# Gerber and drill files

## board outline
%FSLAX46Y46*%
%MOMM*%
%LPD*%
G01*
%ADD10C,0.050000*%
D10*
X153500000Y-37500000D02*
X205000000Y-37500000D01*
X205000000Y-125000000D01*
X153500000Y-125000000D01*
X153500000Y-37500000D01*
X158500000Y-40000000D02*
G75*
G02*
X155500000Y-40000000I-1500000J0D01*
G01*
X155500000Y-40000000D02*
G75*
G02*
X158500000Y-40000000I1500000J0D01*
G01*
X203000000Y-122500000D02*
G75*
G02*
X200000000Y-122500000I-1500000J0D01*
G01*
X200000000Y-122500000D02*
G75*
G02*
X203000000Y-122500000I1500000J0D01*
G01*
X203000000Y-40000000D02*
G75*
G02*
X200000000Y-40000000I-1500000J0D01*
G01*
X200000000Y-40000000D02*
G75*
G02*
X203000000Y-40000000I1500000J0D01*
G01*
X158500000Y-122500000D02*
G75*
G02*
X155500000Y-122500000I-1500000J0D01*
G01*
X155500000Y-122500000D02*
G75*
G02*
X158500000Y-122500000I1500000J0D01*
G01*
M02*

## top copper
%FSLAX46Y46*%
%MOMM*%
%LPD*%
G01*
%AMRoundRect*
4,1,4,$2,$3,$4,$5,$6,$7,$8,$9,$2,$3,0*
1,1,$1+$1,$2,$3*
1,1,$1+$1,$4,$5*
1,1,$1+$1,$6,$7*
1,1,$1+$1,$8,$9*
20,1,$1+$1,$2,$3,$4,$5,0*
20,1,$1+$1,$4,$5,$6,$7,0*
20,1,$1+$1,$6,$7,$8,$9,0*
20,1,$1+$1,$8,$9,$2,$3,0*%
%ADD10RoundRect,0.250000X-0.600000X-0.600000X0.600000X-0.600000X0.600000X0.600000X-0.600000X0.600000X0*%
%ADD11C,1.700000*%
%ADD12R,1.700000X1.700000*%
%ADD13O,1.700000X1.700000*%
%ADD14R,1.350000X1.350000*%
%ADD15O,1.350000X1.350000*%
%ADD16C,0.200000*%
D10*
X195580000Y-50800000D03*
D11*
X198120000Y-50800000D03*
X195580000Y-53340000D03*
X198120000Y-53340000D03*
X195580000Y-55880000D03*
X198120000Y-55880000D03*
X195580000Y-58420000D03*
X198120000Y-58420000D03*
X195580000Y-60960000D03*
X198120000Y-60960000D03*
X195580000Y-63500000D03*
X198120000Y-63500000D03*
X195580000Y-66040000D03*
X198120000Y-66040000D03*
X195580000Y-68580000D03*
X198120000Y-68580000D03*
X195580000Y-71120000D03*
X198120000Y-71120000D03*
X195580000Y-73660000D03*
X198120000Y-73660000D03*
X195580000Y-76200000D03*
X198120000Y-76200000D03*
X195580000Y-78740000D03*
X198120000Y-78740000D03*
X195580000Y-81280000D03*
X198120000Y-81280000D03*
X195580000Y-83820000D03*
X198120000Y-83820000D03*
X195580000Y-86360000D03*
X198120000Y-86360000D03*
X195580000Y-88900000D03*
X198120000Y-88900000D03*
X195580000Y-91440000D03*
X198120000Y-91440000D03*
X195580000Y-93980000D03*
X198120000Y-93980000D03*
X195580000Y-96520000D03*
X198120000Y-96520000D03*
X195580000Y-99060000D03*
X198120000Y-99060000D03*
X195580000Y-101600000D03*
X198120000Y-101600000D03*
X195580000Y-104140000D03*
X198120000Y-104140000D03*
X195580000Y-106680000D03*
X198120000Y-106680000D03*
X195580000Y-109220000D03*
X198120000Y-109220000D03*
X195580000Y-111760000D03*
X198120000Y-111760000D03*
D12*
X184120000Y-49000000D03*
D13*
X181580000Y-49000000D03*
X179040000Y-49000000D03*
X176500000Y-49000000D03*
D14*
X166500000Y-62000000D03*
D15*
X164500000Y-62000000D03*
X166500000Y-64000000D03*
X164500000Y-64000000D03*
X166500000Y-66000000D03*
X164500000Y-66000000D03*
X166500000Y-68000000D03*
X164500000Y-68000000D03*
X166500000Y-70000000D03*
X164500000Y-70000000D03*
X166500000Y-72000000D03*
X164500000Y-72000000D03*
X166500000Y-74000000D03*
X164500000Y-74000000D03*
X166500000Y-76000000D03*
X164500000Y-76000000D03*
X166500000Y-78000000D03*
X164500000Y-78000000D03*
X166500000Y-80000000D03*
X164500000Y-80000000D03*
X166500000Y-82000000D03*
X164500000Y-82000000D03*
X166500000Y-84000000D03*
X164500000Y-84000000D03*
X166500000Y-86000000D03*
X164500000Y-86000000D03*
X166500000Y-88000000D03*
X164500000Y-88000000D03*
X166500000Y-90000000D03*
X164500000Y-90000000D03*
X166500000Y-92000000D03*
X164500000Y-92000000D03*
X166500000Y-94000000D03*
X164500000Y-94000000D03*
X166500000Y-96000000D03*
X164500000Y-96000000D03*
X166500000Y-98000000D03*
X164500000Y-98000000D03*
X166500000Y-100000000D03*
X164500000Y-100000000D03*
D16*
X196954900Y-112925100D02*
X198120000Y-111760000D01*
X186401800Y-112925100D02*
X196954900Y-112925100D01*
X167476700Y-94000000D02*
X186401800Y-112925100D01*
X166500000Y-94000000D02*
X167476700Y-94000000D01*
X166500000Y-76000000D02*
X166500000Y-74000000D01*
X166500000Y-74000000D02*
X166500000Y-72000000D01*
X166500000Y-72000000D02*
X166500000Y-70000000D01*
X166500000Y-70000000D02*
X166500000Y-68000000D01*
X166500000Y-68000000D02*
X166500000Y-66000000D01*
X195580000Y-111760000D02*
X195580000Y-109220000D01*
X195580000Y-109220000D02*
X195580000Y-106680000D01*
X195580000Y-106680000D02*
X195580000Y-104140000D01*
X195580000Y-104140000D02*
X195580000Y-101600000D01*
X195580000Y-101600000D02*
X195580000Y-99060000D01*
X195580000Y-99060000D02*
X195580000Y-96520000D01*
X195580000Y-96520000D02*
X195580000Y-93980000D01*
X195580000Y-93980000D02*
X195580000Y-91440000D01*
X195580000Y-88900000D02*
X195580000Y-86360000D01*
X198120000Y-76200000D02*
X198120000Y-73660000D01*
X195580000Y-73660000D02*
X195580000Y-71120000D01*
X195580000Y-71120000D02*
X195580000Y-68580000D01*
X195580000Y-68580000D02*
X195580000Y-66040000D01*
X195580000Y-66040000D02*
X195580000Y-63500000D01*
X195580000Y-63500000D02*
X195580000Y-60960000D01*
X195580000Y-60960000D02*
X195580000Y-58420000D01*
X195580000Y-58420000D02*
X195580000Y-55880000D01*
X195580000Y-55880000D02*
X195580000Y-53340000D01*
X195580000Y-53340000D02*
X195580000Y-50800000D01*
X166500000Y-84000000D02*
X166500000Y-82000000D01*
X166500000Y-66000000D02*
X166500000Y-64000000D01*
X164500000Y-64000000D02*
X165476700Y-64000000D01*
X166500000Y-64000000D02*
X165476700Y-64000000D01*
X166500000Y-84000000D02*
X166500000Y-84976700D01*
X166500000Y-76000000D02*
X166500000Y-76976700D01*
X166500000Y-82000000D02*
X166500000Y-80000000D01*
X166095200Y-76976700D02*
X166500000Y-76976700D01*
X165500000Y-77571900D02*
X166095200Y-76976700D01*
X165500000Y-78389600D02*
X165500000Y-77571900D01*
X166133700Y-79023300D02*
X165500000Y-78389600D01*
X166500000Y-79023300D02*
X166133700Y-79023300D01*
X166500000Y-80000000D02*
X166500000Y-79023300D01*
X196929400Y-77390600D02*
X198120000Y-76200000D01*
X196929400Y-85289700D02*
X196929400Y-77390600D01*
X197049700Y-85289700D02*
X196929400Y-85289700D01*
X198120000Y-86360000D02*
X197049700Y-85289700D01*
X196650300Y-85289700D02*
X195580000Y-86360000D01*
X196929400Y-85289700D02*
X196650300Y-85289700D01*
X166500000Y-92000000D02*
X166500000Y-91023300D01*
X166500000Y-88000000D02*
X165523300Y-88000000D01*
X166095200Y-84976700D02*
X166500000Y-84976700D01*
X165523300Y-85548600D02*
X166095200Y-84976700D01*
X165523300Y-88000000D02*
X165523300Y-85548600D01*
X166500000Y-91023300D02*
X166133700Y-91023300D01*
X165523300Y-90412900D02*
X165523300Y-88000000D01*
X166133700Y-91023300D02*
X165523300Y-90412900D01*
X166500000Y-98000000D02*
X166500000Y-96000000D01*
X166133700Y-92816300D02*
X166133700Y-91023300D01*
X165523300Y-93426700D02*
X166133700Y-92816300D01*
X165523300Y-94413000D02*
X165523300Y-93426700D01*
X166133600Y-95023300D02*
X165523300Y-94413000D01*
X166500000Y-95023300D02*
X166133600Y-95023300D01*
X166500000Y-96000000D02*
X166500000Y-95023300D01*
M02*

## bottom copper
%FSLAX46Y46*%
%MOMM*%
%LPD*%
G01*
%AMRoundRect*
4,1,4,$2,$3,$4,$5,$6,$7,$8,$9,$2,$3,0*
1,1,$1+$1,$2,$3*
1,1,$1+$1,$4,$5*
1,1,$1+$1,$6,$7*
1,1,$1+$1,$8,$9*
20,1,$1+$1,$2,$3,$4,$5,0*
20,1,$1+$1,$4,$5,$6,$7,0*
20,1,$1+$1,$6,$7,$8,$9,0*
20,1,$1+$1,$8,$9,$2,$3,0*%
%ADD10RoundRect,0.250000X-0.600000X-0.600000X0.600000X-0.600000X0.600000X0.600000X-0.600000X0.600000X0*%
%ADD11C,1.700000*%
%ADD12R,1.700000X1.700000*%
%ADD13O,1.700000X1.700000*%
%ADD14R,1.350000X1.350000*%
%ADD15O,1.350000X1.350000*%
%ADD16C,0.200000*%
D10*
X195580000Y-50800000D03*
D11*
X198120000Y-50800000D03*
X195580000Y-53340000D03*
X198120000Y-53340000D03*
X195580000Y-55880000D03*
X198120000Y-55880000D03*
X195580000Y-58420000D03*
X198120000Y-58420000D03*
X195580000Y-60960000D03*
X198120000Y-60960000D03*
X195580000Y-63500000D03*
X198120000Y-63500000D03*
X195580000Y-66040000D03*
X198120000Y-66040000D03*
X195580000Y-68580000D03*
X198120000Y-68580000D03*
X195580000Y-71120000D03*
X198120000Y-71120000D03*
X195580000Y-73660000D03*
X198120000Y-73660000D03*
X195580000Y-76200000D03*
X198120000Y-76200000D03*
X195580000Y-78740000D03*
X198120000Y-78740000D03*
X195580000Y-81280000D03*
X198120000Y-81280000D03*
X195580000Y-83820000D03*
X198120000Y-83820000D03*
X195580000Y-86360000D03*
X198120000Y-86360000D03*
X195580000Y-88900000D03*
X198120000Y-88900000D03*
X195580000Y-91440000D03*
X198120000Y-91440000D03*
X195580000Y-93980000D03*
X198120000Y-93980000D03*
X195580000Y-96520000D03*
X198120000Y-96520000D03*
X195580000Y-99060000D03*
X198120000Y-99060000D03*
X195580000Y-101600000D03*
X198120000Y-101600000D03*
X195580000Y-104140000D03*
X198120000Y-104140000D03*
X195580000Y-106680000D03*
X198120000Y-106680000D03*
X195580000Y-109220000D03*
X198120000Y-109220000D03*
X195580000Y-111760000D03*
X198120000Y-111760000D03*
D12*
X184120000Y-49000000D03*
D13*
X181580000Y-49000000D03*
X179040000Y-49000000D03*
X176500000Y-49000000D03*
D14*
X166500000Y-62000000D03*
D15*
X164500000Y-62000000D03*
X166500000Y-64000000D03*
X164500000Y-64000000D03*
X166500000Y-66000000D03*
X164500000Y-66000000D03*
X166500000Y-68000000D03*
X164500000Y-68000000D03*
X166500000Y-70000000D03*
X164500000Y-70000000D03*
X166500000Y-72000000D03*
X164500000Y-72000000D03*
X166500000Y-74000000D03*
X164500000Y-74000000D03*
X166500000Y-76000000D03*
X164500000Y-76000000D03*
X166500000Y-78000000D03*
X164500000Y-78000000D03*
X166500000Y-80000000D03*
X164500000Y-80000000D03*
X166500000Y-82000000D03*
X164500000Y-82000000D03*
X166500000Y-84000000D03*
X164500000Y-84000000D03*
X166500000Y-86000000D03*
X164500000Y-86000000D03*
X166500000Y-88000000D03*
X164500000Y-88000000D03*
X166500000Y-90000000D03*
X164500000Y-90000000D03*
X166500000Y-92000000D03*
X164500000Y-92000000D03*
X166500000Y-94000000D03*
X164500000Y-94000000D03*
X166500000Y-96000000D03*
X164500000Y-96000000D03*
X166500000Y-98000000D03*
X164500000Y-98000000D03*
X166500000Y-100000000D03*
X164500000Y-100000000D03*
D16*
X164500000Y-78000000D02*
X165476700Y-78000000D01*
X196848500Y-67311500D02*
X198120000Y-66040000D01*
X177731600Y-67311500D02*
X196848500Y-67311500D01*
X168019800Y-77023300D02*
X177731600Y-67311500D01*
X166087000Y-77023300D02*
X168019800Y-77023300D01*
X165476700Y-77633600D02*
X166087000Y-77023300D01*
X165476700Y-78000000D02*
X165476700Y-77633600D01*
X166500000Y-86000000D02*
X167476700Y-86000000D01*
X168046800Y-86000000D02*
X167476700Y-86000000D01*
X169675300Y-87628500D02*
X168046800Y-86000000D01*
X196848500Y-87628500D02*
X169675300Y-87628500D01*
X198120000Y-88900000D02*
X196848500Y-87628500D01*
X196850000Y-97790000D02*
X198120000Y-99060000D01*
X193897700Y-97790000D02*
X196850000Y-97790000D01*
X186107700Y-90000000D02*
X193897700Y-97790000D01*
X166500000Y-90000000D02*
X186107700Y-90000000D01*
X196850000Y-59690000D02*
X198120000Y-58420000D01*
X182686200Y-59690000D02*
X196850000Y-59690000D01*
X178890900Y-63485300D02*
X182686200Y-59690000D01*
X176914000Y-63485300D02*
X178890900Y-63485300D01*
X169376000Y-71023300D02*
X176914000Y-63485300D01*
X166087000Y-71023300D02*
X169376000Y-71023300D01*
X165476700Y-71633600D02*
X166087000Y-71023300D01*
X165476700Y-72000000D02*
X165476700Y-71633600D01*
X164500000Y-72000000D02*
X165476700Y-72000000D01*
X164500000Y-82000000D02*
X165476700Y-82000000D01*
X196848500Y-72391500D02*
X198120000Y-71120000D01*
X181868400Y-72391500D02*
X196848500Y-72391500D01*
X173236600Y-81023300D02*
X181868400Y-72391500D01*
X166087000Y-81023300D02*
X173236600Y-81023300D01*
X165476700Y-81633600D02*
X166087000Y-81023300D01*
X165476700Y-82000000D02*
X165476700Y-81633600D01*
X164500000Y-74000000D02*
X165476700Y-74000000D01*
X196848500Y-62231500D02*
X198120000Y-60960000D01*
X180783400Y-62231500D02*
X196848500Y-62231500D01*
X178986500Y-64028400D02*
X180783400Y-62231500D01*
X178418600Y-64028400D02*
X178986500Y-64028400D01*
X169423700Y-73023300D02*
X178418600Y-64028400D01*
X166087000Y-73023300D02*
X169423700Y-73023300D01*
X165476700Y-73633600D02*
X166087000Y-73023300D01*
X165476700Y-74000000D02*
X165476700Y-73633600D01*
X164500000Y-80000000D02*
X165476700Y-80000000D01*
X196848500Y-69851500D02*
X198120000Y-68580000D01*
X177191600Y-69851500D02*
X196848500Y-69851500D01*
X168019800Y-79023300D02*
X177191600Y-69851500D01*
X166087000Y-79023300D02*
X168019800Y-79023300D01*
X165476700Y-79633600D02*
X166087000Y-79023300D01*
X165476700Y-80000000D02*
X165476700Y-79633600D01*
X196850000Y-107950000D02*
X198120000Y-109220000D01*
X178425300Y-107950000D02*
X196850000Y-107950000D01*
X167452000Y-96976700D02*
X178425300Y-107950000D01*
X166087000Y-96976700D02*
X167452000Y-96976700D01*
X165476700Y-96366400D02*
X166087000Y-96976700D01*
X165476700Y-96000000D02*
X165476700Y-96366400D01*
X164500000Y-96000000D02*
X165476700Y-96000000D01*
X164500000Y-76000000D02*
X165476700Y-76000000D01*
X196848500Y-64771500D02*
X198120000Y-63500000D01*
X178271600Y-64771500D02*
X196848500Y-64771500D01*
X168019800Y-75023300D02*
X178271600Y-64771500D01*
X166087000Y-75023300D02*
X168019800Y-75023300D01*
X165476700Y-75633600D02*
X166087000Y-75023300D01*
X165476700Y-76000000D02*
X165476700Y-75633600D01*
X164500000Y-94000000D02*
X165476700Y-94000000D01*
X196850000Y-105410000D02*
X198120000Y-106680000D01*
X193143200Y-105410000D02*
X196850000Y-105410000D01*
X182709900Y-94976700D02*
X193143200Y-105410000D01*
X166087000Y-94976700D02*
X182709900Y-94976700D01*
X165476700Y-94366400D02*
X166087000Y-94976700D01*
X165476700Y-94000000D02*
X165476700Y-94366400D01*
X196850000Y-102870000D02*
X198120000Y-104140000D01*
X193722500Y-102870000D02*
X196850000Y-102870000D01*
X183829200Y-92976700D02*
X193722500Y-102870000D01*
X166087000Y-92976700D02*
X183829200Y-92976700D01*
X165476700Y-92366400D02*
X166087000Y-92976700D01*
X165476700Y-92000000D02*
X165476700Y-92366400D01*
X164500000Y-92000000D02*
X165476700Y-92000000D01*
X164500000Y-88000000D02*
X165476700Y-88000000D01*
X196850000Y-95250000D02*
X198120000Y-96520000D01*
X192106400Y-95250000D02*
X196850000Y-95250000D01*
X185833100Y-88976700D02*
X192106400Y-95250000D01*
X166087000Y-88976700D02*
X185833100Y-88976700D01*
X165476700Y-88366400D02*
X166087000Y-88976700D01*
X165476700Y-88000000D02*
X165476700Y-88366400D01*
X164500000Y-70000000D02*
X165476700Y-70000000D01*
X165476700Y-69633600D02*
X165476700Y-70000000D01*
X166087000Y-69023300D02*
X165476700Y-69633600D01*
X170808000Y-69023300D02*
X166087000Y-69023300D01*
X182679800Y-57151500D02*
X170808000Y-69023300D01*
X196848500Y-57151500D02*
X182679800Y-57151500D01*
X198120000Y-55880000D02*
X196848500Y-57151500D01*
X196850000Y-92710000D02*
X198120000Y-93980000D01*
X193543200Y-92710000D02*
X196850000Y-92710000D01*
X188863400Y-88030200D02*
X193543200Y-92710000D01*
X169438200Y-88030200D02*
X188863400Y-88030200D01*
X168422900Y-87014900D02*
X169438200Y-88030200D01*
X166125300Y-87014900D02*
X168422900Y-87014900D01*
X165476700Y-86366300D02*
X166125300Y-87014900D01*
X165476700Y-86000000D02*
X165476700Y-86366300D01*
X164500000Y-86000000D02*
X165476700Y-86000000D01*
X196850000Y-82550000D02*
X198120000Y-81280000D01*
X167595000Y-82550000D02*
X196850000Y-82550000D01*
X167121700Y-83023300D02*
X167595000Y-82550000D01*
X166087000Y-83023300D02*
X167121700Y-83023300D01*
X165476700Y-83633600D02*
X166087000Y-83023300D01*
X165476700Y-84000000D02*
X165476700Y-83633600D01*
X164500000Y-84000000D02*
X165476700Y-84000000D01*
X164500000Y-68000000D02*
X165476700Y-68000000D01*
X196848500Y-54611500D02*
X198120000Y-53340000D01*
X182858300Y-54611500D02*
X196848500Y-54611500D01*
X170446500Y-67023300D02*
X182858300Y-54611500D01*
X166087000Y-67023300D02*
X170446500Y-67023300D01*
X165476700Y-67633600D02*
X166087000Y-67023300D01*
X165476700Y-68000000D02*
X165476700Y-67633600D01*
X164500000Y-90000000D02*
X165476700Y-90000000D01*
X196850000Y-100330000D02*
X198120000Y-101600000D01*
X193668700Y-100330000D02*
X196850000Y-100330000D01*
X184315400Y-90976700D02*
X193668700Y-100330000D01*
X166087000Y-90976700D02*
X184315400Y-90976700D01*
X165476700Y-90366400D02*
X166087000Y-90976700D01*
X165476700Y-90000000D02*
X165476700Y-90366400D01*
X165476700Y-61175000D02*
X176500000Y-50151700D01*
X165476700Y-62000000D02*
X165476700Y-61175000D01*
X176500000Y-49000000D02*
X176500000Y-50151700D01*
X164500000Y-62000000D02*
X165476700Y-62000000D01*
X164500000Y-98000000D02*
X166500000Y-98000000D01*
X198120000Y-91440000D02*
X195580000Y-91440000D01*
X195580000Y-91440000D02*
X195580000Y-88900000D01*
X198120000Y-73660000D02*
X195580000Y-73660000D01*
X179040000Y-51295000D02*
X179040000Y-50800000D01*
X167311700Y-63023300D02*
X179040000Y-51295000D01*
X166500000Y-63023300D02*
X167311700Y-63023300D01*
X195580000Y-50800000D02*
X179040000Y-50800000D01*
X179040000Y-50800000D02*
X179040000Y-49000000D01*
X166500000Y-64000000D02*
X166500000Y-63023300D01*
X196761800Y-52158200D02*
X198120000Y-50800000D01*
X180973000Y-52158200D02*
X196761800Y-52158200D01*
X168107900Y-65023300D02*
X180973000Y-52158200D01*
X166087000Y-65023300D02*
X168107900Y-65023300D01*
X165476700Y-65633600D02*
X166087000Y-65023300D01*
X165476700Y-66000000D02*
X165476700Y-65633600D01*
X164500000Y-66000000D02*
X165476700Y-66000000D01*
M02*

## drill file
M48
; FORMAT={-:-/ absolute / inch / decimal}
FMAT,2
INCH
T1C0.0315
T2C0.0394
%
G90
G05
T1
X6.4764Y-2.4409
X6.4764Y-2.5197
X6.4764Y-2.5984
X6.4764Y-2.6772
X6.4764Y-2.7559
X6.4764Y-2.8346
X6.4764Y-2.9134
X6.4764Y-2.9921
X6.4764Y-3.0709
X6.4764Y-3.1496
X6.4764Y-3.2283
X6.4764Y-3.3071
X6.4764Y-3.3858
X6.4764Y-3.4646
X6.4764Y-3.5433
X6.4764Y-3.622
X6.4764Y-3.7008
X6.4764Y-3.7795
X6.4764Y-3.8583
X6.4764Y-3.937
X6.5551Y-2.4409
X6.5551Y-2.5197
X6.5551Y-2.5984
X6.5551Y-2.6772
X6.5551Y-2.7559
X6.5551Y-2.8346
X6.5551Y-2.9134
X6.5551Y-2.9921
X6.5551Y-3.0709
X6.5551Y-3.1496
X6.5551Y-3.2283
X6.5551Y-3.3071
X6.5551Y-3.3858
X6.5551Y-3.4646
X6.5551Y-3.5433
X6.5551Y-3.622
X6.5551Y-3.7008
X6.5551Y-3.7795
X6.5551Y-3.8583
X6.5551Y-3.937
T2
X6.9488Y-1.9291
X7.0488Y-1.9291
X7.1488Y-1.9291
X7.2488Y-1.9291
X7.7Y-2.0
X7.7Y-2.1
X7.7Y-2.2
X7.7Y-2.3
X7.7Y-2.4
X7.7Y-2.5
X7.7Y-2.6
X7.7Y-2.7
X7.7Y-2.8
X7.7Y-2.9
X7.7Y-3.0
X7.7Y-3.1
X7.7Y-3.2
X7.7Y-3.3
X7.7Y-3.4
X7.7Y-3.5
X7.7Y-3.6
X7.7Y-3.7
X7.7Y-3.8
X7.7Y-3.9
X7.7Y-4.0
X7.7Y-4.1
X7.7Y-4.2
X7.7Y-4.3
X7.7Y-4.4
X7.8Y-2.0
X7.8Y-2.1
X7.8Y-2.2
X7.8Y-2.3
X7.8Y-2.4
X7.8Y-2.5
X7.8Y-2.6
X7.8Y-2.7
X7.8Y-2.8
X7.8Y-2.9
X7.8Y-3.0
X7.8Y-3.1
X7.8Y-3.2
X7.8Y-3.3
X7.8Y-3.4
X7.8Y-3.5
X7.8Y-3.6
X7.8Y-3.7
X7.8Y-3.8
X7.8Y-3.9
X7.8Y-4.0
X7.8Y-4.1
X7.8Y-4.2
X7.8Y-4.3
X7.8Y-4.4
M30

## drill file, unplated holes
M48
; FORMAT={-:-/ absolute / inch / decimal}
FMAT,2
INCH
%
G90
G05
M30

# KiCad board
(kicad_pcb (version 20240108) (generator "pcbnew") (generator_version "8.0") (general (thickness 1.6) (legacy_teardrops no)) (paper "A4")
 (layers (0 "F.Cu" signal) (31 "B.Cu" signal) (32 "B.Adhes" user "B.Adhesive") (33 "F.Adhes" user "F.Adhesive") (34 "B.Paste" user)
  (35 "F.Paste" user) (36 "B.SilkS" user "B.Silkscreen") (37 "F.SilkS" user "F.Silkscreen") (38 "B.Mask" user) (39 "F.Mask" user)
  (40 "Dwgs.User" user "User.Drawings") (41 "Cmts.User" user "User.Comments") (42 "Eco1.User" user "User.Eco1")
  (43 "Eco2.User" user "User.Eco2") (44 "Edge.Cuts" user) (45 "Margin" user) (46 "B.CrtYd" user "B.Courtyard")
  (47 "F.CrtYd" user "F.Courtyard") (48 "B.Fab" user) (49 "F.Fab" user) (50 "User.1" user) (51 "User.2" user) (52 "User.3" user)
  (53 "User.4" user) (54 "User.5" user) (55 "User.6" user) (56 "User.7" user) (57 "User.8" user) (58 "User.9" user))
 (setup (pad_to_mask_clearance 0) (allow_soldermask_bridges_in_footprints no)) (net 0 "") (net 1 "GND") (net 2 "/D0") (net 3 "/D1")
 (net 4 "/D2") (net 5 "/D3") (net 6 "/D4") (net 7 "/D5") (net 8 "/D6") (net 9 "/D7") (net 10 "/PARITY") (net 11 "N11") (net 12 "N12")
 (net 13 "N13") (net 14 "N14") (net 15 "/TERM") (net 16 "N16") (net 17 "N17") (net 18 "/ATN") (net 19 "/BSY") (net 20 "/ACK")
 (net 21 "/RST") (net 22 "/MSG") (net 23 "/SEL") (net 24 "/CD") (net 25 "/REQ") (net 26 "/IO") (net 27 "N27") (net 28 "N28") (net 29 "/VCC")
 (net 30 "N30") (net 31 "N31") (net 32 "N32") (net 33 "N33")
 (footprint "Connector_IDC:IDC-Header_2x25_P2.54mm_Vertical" (layer "F.Cu") (at 195.58 50.8)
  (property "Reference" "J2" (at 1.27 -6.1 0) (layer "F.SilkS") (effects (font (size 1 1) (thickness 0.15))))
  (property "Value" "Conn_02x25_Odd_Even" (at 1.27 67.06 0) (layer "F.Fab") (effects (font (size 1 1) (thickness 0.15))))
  (pad "1" thru_hole roundrect (at 0 0) (size 1.7 1.7) (drill 1) (layers "*.Cu" "*.Mask") (remove_unused_layers no)
   (roundrect_rratio 0.147059) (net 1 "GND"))
  (pad "2" thru_hole circle (at 2.54 0) (size 1.7 1.7) (drill 1) (layers "*.Cu" "*.Mask") (remove_unused_layers no) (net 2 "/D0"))
  (pad "3" thru_hole circle (at 0 2.54) (size 1.7 1.7) (drill 1) (layers "*.Cu" "*.Mask") (remove_unused_layers no) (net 1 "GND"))
  (pad "4" thru_hole circle (at 2.54 2.54) (size 1.7 1.7) (drill 1) (layers "*.Cu" "*.Mask") (remove_unused_layers no) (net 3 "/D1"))
  (pad "5" thru_hole circle (at 0 5.08) (size 1.7 1.7) (drill 1) (layers "*.Cu" "*.Mask") (remove_unused_layers no) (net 1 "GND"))
  (pad "6" thru_hole circle (at 2.54 5.08) (size 1.7 1.7) (drill 1) (layers "*.Cu" "*.Mask") (remove_unused_layers no) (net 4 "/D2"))
  (pad "7" thru_hole circle (at 0 7.62) (size 1.7 1.7) (drill 1) (layers "*.Cu" "*.Mask") (remove_unused_layers no) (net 1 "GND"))
  (pad "8" thru_hole circle (at 2.54 7.62) (size 1.7 1.7) (drill 1) (layers "*.Cu" "*.Mask") (remove_unused_layers no) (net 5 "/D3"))
  (pad "9" thru_hole circle (at 0 10.16) (size 1.7 1.7) (drill 1) (layers "*.Cu" "*.Mask") (remove_unused_layers no) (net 1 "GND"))
  (pad "10" thru_hole circle (at 2.54 10.16) (size 1.7 1.7) (drill 1) (layers "*.Cu" "*.Mask") (remove_unused_layers no) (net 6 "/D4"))
  (pad "11" thru_hole circle (at 0 12.7) (size 1.7 1.7) (drill 1) (layers "*.Cu" "*.Mask") (remove_unused_layers no) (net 1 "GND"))
  (pad "12" thru_hole circle (at 2.54 12.7) (size 1.7 1.7) (drill 1) (layers "*.Cu" "*.Mask") (remove_unused_layers no) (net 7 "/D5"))
  (pad "13" thru_hole circle (at 0 15.24) (size 1.7 1.7) (drill 1) (layers "*.Cu" "*.Mask") (remove_unused_layers no) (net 1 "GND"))
  (pad "14" thru_hole circle (at 2.54 15.24) (size 1.7 1.7) (drill 1) (layers "*.Cu" "*.Mask") (remove_unused_layers no) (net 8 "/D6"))
  (pad "15" thru_hole circle (at 0 17.78) (size 1.7 1.7) (drill 1) (layers "*.Cu" "*.Mask") (remove_unused_layers no) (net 1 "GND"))
  (pad "16" thru_hole circle (at 2.54 17.78) (size 1.7 1.7) (drill 1) (layers "*.Cu" "*.Mask") (remove_unused_layers no) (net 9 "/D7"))
  (pad "17" thru_hole circle (at 0 20.32) (size 1.7 1.7) (drill 1) (layers "*.Cu" "*.Mask") (remove_unused_layers no) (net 1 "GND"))
  (pad "18" thru_hole circle (at 2.54 20.32) (size 1.7 1.7) (drill 1) (layers "*.Cu" "*.Mask") (remove_unused_layers no) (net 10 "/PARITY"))
  (pad "19" thru_hole circle (at 0 22.86) (size 1.7 1.7) (drill 1) (layers "*.Cu" "*.Mask") (remove_unused_layers no) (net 1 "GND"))
  (pad "20" thru_hole circle (at 2.54 22.86) (size 1.7 1.7) (drill 1) (layers "*.Cu" "*.Mask") (remove_unused_layers no) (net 1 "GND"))
  (pad "21" thru_hole circle (at 0 25.4) (size 1.7 1.7) (drill 1) (layers "*.Cu" "*.Mask") (remove_unused_layers no) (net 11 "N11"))
  (pad "22" thru_hole circle (at 2.54 25.4) (size 1.7 1.7) (drill 1) (layers "*.Cu" "*.Mask") (remove_unused_layers no) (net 1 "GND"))
  (pad "23" thru_hole circle (at 0 27.94) (size 1.7 1.7) (drill 1) (layers "*.Cu" "*.Mask") (remove_unused_layers no) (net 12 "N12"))
  (pad "24" thru_hole circle (at 2.54 27.94) (size 1.7 1.7) (drill 1) (layers "*.Cu" "*.Mask") (remove_unused_layers no) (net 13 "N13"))
  (pad "25" thru_hole circle (at 0 30.48) (size 1.7 1.7) (drill 1) (layers "*.Cu" "*.Mask") (remove_unused_layers no) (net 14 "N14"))
  (pad "26" thru_hole circle (at 2.54 30.48) (size 1.7 1.7) (drill 1) (layers "*.Cu" "*.Mask") (remove_unused_layers no) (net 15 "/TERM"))
  (pad "27" thru_hole circle (at 0 33.02) (size 1.7 1.7) (drill 1) (layers "*.Cu" "*.Mask") (remove_unused_layers no) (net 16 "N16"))
  (pad "28" thru_hole circle (at 2.54 33.02) (size 1.7 1.7) (drill 1) (layers "*.Cu" "*.Mask") (remove_unused_layers no) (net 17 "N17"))
  (pad "29" thru_hole circle (at 0 35.56) (size 1.7 1.7) (drill 1) (layers "*.Cu" "*.Mask") (remove_unused_layers no) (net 1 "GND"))
  (pad "30" thru_hole circle (at 2.54 35.56) (size 1.7 1.7) (drill 1) (layers "*.Cu" "*.Mask") (remove_unused_layers no) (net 1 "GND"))
  (pad "31" thru_hole circle (at 0 38.1) (size 1.7 1.7) (drill 1) (layers "*.Cu" "*.Mask") (remove_unused_layers no) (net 1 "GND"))
  (pad "32" thru_hole circle (at 2.54 38.1) (size 1.7 1.7) (drill 1) (layers "*.Cu" "*.Mask") (remove_unused_layers no) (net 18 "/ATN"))
  (pad "33" thru_hole circle (at 0 40.64) (size 1.7 1.7) (drill 1) (layers "*.Cu" "*.Mask") (remove_unused_layers no) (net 1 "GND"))
  (pad "34" thru_hole circle (at 2.54 40.64) (size 1.7 1.7) (drill 1) (layers "*.Cu" "*.Mask") (remove_unused_layers no) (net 1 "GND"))
  (pad "35" thru_hole circle (at 0 43.18) (size 1.7 1.7) (drill 1) (layers "*.Cu" "*.Mask") (remove_unused_layers no) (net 1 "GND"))
  (pad "36" thru_hole circle (at 2.54 43.18) (size 1.7 1.7) (drill 1) (layers "*.Cu" "*.Mask") (remove_unused_layers no) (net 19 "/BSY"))
  (pad "37" thru_hole circle (at 0 45.72) (size 1.7 1.7) (drill 1) (layers "*.Cu" "*.Mask") (remove_unused_layers no) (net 1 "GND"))
  (pad "38" thru_hole circle (at 2.54 45.72) (size 1.7 1.7) (drill 1) (layers "*.Cu" "*.Mask") (remove_unused_layers no) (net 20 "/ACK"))
  (pad "39" thru_hole circle (at 0 48.26) (size 1.7 1.7) (drill 1) (layers "*.Cu" "*.Mask") (remove_unused_layers no) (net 1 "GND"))
  (pad "40" thru_hole circle (at 2.54 48.26) (size 1.7 1.7) (drill 1) (layers "*.Cu" "*.Mask") (remove_unused_layers no) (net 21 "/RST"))
  (pad "41" thru_hole circle (at 0 50.8) (size 1.7 1.7) (drill 1) (layers "*.Cu" "*.Mask") (remove_unused_layers no) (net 1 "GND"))
  (pad "42" thru_hole circle (at 2.54 50.8) (size 1.7 1.7) (drill 1) (layers "*.Cu" "*.Mask") (remove_unused_layers no) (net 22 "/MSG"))
  (pad "43" thru_hole circle (at 0 53.34) (size 1.7 1.7) (drill 1) (layers "*.Cu" "*.Mask") (remove_unused_layers no) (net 1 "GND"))
  (pad "44" thru_hole circle (at 2.54 53.34) (size 1.7 1.7) (drill 1) (layers "*.Cu" "*.Mask") (remove_unused_layers no) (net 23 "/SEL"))
  (pad "45" thru_hole circle (at 0 55.88) (size 1.7 1.7) (drill 1) (layers "*.Cu" "*.Mask") (remove_unused_layers no) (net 1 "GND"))
  (pad "46" thru_hole circle (at 2.54 55.88) (size 1.7 1.7) (drill 1) (layers "*.Cu" "*.Mask") (remove_unused_layers no) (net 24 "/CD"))
  (pad "47" thru_hole circle (at 0 58.42) (size 1.7 1.7) (drill 1) (layers "*.Cu" "*.Mask") (remove_unused_layers no) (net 1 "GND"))
  (pad "48" thru_hole circle (at 2.54 58.42) (size 1.7 1.7) (drill 1) (layers "*.Cu" "*.Mask") (remove_unused_layers no) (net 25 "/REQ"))
  (pad "49" thru_hole circle (at 0 60.96) (size 1.7 1.7) (drill 1) (layers "*.Cu" "*.Mask") (remove_unused_layers no) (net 1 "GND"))
  (pad "50" thru_hole circle (at 2.54 60.96) (size 1.7 1.7) (drill 1) (layers "*.Cu" "*.Mask") (remove_unused_layers no) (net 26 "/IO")))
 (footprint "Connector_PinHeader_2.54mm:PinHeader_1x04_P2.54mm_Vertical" (layer "F.Cu") (at 184.12 49 -90)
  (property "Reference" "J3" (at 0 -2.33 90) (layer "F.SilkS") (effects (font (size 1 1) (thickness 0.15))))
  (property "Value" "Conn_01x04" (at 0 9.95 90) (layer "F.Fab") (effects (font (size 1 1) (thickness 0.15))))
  (pad "1" thru_hole rect (at 0 0 270) (size 1.7 1.7) (drill 1) (layers "*.Cu" "*.Mask") (remove_unused_layers no) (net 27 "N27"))
  (pad "2" thru_hole oval (at 0 2.54 270) (size 1.7 1.7) (drill 1) (layers "*.Cu" "*.Mask") (remove_unused_layers no) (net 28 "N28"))
  (pad "3" thru_hole oval (at 0 5.08 270) (size 1.7 1.7) (drill 1) (layers "*.Cu" "*.Mask") (remove_unused_layers no) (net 1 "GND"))
  (pad "4" thru_hole oval (at 0 7.62 270) (size 1.7 1.7) (drill 1) (layers "*.Cu" "*.Mask") (remove_unused_layers no) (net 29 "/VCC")))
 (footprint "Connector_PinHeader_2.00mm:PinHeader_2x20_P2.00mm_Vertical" (layer "B.Cu") (at 166.5 62 180)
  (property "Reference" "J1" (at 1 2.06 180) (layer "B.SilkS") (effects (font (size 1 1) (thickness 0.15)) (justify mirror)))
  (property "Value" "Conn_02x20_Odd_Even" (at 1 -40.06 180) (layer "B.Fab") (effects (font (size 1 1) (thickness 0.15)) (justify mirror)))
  (pad "1" thru_hole rect (at 0 0 180) (size 1.35 1.35) (drill 0.8) (layers "*.Cu" "*.Mask") (remove_unused_layers no) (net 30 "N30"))
  (pad "2" thru_hole oval (at 2 0 180) (size 1.35 1.35) (drill 0.8) (layers "*.Cu" "*.Mask") (remove_unused_layers no) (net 29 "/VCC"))
  (pad "3" thru_hole oval (at 0 -2 180) (size 1.35 1.35) (drill 0.8) (layers "*.Cu" "*.Mask") (remove_unused_layers no) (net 1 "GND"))
  (pad "4" thru_hole oval (at 2 -2 180) (size 1.35 1.35) (drill 0.8) (layers "*.Cu" "*.Mask") (remove_unused_layers no) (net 1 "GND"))
  (pad "5" thru_hole oval (at 0 -4 180) (size 1.35 1.35) (drill 0.8) (layers "*.Cu" "*.Mask") (remove_unused_layers no) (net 1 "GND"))
  (pad "6" thru_hole oval (at 2 -4 180) (size 1.35 1.35) (drill 0.8) (layers "*.Cu" "*.Mask") (remove_unused_layers no) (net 2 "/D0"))
  (pad "7" thru_hole oval (at 0 -6 180) (size 1.35 1.35) (drill 0.8) (layers "*.Cu" "*.Mask") (remove_unused_layers no) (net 1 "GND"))
  (pad "8" thru_hole oval (at 2 -6 180) (size 1.35 1.35) (drill 0.8) (layers "*.Cu" "*.Mask") (remove_unused_layers no) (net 3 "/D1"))
  (pad "9" thru_hole oval (at 0 -8 180) (size 1.35 1.35) (drill 0.8) (layers "*.Cu" "*.Mask") (remove_unused_layers no) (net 1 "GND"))
  (pad "10" thru_hole oval (at 2 -8 180) (size 1.35 1.35) (drill 0.8) (layers "*.Cu" "*.Mask") (remove_unused_layers no) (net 4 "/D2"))
  (pad "11" thru_hole oval (at 0 -10 180) (size 1.35 1.35) (drill 0.8) (layers "*.Cu" "*.Mask") (remove_unused_layers no) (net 1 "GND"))
  (pad "12" thru_hole oval (at 2 -10 180) (size 1.35 1.35) (drill 0.8) (layers "*.Cu" "*.Mask") (remove_unused_layers no) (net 5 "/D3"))
  (pad "13" thru_hole oval (at 0 -12 180) (size 1.35 1.35) (drill 0.8) (layers "*.Cu" "*.Mask") (remove_unused_layers no) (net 1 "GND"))
  (pad "14" thru_hole oval (at 2 -12 180) (size 1.35 1.35) (drill 0.8) (layers "*.Cu" "*.Mask") (remove_unused_layers no) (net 6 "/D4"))
  (pad "15" thru_hole oval (at 0 -14 180) (size 1.35 1.35) (drill 0.8) (layers "*.Cu" "*.Mask") (remove_unused_layers no) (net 1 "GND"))
  (pad "16" thru_hole oval (at 2 -14 180) (size 1.35 1.35) (drill 0.8) (layers "*.Cu" "*.Mask") (remove_unused_layers no) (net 7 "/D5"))
  (pad "17" thru_hole oval (at 0 -16 180) (size 1.35 1.35) (drill 0.8) (layers "*.Cu" "*.Mask") (remove_unused_layers no) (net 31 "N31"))
  (pad "18" thru_hole oval (at 2 -16 180) (size 1.35 1.35) (drill 0.8) (layers "*.Cu" "*.Mask") (remove_unused_layers no) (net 8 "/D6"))
  (pad "19" thru_hole oval (at 0 -18 180) (size 1.35 1.35) (drill 0.8) (layers "*.Cu" "*.Mask") (remove_unused_layers no) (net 1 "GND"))
  (pad "20" thru_hole oval (at 2 -18 180) (size 1.35 1.35) (drill 0.8) (layers "*.Cu" "*.Mask") (remove_unused_layers no) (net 9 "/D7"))
  (pad "21" thru_hole oval (at 0 -20 180) (size 1.35 1.35) (drill 0.8) (layers "*.Cu" "*.Mask") (remove_unused_layers no) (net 1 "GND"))
  (pad "22" thru_hole oval (at 2 -20 180) (size 1.35 1.35) (drill 0.8) (layers "*.Cu" "*.Mask") (remove_unused_layers no) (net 10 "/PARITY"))
  (pad "23" thru_hole oval (at 0 -22 180) (size 1.35 1.35) (drill 0.8) (layers "*.Cu" "*.Mask") (remove_unused_layers no) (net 1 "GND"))
  (pad "24" thru_hole oval (at 2 -22 180) (size 1.35 1.35) (drill 0.8) (layers "*.Cu" "*.Mask") (remove_unused_layers no) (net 15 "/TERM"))
  (pad "25" thru_hole oval (at 0 -24 180) (size 1.35 1.35) (drill 0.8) (layers "*.Cu" "*.Mask") (remove_unused_layers no) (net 18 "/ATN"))
  (pad "26" thru_hole oval (at 2 -24 180) (size 1.35 1.35) (drill 0.8) (layers "*.Cu" "*.Mask") (remove_unused_layers no) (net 19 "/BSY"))
  (pad "27" thru_hole oval (at 0 -26 180) (size 1.35 1.35) (drill 0.8) (layers "*.Cu" "*.Mask") (remove_unused_layers no) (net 1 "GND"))
  (pad "28" thru_hole oval (at 2 -26 180) (size 1.35 1.35) (drill 0.8) (layers "*.Cu" "*.Mask") (remove_unused_layers no) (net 20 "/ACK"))
  (pad "29" thru_hole oval (at 0 -28 180) (size 1.35 1.35) (drill 0.8) (layers "*.Cu" "*.Mask") (remove_unused_layers no) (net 21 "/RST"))
  (pad "30" thru_hole oval (at 2 -28 180) (size 1.35 1.35) (drill 0.8) (layers "*.Cu" "*.Mask") (remove_unused_layers no) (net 22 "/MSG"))
  (pad "31" thru_hole oval (at 0 -30 180) (size 1.35 1.35) (drill 0.8) (layers "*.Cu" "*.Mask") (remove_unused_layers no) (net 1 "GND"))
  (pad "32" thru_hole oval (at 2 -30 180) (size 1.35 1.35) (drill 0.8) (layers "*.Cu" "*.Mask") (remove_unused_layers no) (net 23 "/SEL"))
  (pad "33" thru_hole oval (at 0 -32 180) (size 1.35 1.35) (drill 0.8) (layers "*.Cu" "*.Mask") (remove_unused_layers no) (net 26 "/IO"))
  (pad "34" thru_hole oval (at 2 -32 180) (size 1.35 1.35) (drill 0.8) (layers "*.Cu" "*.Mask") (remove_unused_layers no) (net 24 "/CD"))
  (pad "35" thru_hole oval (at 0 -34 180) (size 1.35 1.35) (drill 0.8) (layers "*.Cu" "*.Mask") (remove_unused_layers no) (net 1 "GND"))
  (pad "36" thru_hole oval (at 2 -34 180) (size 1.35 1.35) (drill 0.8) (layers "*.Cu" "*.Mask") (remove_unused_layers no) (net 25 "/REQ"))
  (pad "37" thru_hole oval (at 0 -36 180) (size 1.35 1.35) (drill 0.8) (layers "*.Cu" "*.Mask") (remove_unused_layers no) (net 1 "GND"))
  (pad "38" thru_hole oval (at 2 -36 180) (size 1.35 1.35) (drill 0.8) (layers "*.Cu" "*.Mask") (remove_unused_layers no) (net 1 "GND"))
  (pad "39" thru_hole oval (at 0 -38 180) (size 1.35 1.35) (drill 0.8) (layers "*.Cu" "*.Mask") (remove_unused_layers no) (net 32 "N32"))
  (pad "40" thru_hole oval (at 2 -38 180) (size 1.35 1.35) (drill 0.8) (layers "*.Cu" "*.Mask") (remove_unused_layers no) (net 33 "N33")))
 (gr_rect (start 153.5 37.5) (end 205 125) (stroke (width 0.05) (type default)) (fill none) (layer "Edge.Cuts"))
 (gr_circle (center 157 40) (end 155.5 40) (stroke (width 0.05) (type default)) (fill none) (layer "Edge.Cuts"))
 (gr_circle (center 201.5 122.5) (end 200 122.5) (stroke (width 0.05) (type default)) (fill none) (layer "Edge.Cuts"))
 (gr_circle (center 201.5 40) (end 200 40) (stroke (width 0.05) (type default)) (fill none) (layer "Edge.Cuts"))
 (gr_circle (center 157 122.5) (end 155.5 122.5) (stroke (width 0.05) (type default)) (fill none) (layer "Edge.Cuts"))
 (segment (start 196.7618 52.1582) (end 198.12 50.8) (width 0.2) (layer "B.Cu") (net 2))
 (segment (start 180.973 52.1582) (end 196.7618 52.1582) (width 0.2) (layer "B.Cu") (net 2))
 (segment (start 165.4767 66) (end 165.4767 65.6336) (width 0.2) (layer "B.Cu") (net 2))
 (segment (start 168.1079 65.0233) (end 180.973 52.1582) (width 0.2) (layer "B.Cu") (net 2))
 (segment (start 165.4767 65.6336) (end 166.087 65.0233) (width 0.2) (layer "B.Cu") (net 2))
 (segment (start 164.5 66) (end 165.4767 66) (width 0.2) (layer "B.Cu") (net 2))
 (segment (start 166.087 65.0233) (end 168.1079 65.0233) (width 0.2) (layer "B.Cu") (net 2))
 (segment (start 195.58 68.58) (end 195.58 66.04) (width 0.2) (layer "F.Cu") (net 1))
 (segment (start 197.0497 85.2897) (end 196.9294 85.2897) (width 0.2) (layer "F.Cu") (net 1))
 (segment (start 166.5 95.0233) (end 166.1336 95.0233) (width 0.2) (layer "F.Cu") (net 1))
 (segment (start 195.58 109.22) (end 195.58 106.68) (width 0.2) (layer "F.Cu") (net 1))
 (segment (start 195.58 53.34) (end 195.58 50.8) (width 0.2) (layer "F.Cu") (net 1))
 (segment (start 165.5233 88) (end 165.5233 85.5486) (width 0.2) (layer "F.Cu") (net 1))
 (segment (start 166.5 98) (end 166.5 96) (width 0.2) (layer "F.Cu") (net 1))
 (segment (start 196.9294 85.2897) (end 196.6503 85.2897) (width 0.2) (layer "F.Cu") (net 1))
 (segment (start 166.5 64) (end 165.4767 64) (width 0.2) (layer "F.Cu") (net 1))
 (segment (start 166.5 66) (end 166.5 64) (width 0.2) (layer "F.Cu") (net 1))
 (segment (start 166.5 91.0233) (end 166.1337 91.0233) (width 0.2) (layer "F.Cu") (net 1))
 (segment (start 166.5 84) (end 166.5 82) (width 0.2) (layer "F.Cu") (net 1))
 (segment (start 195.58 111.76) (end 195.58 109.22) (width 0.2) (layer "F.Cu") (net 1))
 (segment (start 166.1336 95.0233) (end 165.5233 94.413) (width 0.2) (layer "F.Cu") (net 1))
 (segment (start 195.58 104.14) (end 195.58 101.6) (width 0.2) (layer "F.Cu") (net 1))
 (segment (start 195.58 99.06) (end 195.58 96.52) (width 0.2) (layer "F.Cu") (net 1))
 (segment (start 195.58 60.96) (end 195.58 58.42) (width 0.2) (layer "F.Cu") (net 1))
 (segment (start 166.0952 76.9767) (end 166.5 76.9767) (width 0.2) (layer "F.Cu") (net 1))
 (segment (start 166.5 76) (end 166.5 74) (width 0.2) (layer "F.Cu") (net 1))
 (segment (start 166.5 96) (end 166.5 95.0233) (width 0.2) (layer "F.Cu") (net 1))
 (segment (start 195.58 88.9) (end 195.58 86.36) (width 0.2) (layer "F.Cu") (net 1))
 (segment (start 166.5 82) (end 166.5 80) (width 0.2) (layer "F.Cu") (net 1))
 (segment (start 198.12 76.2) (end 198.12 73.66) (width 0.2) (layer "F.Cu") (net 1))
 (segment (start 195.58 73.66) (end 195.58 71.12) (width 0.2) (layer "F.Cu") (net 1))
 (segment (start 195.58 58.42) (end 195.58 55.88) (width 0.2) (layer "F.Cu") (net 1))
 (segment (start 195.58 101.6) (end 195.58 99.06) (width 0.2) (layer "F.Cu") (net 1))
 (segment (start 196.9294 85.2897) (end 196.9294 77.3906) (width 0.2) (layer "F.Cu") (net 1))
 (segment (start 166.5 72) (end 166.5 70) (width 0.2) (layer "F.Cu") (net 1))
 (segment (start 198.12 86.36) (end 197.0497 85.2897) (width 0.2) (layer "F.Cu") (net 1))
 (segment (start 165.5 78.3896) (end 165.5 77.5719) (width 0.2) (layer "F.Cu") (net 1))
 (segment (start 195.58 106.68) (end 195.58 104.14) (width 0.2) (layer "F.Cu") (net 1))
 (segment (start 196.9294 77.3906) (end 198.12 76.2) (width 0.2) (layer "F.Cu") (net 1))
 (segment (start 166.1337 92.8163) (end 166.1337 91.0233) (width 0.2) (layer "F.Cu") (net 1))
 (segment (start 166.5 76) (end 166.5 76.9767) (width 0.2) (layer "F.Cu") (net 1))
 (segment (start 166.5 92) (end 166.5 91.0233) (width 0.2) (layer "F.Cu") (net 1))
 (segment (start 165.5233 93.4267) (end 166.1337 92.8163) (width 0.2) (layer "F.Cu") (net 1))
 (segment (start 166.5 88) (end 165.5233 88) (width 0.2) (layer "F.Cu") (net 1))
 (segment (start 195.58 71.12) (end 195.58 68.58) (width 0.2) (layer "F.Cu") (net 1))
 (segment (start 165.5233 90.4129) (end 165.5233 88) (width 0.2) (layer "F.Cu") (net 1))
 (segment (start 195.58 63.5) (end 195.58 60.96) (width 0.2) (layer "F.Cu") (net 1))
 (segment (start 165.5233 94.413) (end 165.5233 93.4267) (width 0.2) (layer "F.Cu") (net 1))
 (segment (start 166.5 68) (end 166.5 66) (width 0.2) (layer "F.Cu") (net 1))
 (segment (start 195.58 55.88) (end 195.58 53.34) (width 0.2) (layer "F.Cu") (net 1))
 (segment (start 165.5233 85.5486) (end 166.0952 84.9767) (width 0.2) (layer "F.Cu") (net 1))
 (segment (start 195.58 96.52) (end 195.58 93.98) (width 0.2) (layer "F.Cu") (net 1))
 (segment (start 195.58 66.04) (end 195.58 63.5) (width 0.2) (layer "F.Cu") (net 1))
 (segment (start 166.1337 79.0233) (end 165.5 78.3896) (width 0.2) (layer "F.Cu") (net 1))
 (segment (start 166.5 80) (end 166.5 79.0233) (width 0.2) (layer "F.Cu") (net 1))
 (segment (start 166.5 70) (end 166.5 68) (width 0.2) (layer "F.Cu") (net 1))
 (segment (start 164.5 64) (end 165.4767 64) (width 0.2) (layer "F.Cu") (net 1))
 (segment (start 196.6503 85.2897) (end 195.58 86.36) (width 0.2) (layer "F.Cu") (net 1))
 (segment (start 195.58 93.98) (end 195.58 91.44) (width 0.2) (layer "F.Cu") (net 1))
 (segment (start 166.1337 91.0233) (end 165.5233 90.4129) (width 0.2) (layer "F.Cu") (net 1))
 (segment (start 166.5 84) (end 166.5 84.9767) (width 0.2) (layer "F.Cu") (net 1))
 (segment (start 166.5 74) (end 166.5 72) (width 0.2) (layer "F.Cu") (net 1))
 (segment (start 166.5 79.0233) (end 166.1337 79.0233) (width 0.2) (layer "F.Cu") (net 1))
 (segment (start 166.0952 84.9767) (end 166.5 84.9767) (width 0.2) (layer "F.Cu") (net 1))
 (segment (start 165.5 77.5719) (end 166.0952 76.9767) (width 0.2) (layer "F.Cu") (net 1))
 (segment (start 166.5 63.0233) (end 167.3117 63.0233) (width 0.2) (layer "B.Cu") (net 1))
 (segment (start 164.5 98) (end 166.5 98) (width 0.2) (layer "B.Cu") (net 1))
 (segment (start 179.04 50.8) (end 179.04 49) (width 0.2) (layer "B.Cu") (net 1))
 (segment (start 198.12 73.66) (end 195.58 73.66) (width 0.2) (layer "B.Cu") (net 1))
 (segment (start 195.58 91.44) (end 195.58 88.9) (width 0.2) (layer "B.Cu") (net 1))
 (segment (start 179.04 51.295) (end 179.04 50.8) (width 0.2) (layer "B.Cu") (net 1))
 (segment (start 166.5 64) (end 166.5 63.0233) (width 0.2) (layer "B.Cu") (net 1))
 (segment (start 195.58 50.8) (end 179.04 50.8) (width 0.2) (layer "B.Cu") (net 1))
 (segment (start 198.12 91.44) (end 195.58 91.44) (width 0.2) (layer "B.Cu") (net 1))
 (segment (start 167.3117 63.0233) (end 179.04 51.295) (width 0.2) (layer "B.Cu") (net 1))
 (segment (start 165.4767 61.175) (end 176.5 50.1517) (width 0.2) (layer "B.Cu") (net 29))
 (segment (start 176.5 49) (end 176.5 50.1517) (width 0.2) (layer "B.Cu") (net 29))
 (segment (start 164.5 62) (end 165.4767 62) (width 0.2) (layer "B.Cu") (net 29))
 (segment (start 165.4767 62) (end 165.4767 61.175) (width 0.2) (layer "B.Cu") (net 29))
 (segment (start 165.4767 90) (end 165.4767 90.3664) (width 0.2) (layer "B.Cu") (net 22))
 (segment (start 165.4767 90.3664) (end 166.087 90.9767) (width 0.2) (layer "B.Cu") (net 22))
 (segment (start 166.087 90.9767) (end 184.3154 90.9767) (width 0.2) (layer "B.Cu") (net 22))
 (segment (start 196.85 100.33) (end 198.12 101.6) (width 0.2) (layer "B.Cu") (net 22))
 (segment (start 193.6687 100.33) (end 196.85 100.33) (width 0.2) (layer "B.Cu") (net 22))
 (segment (start 164.5 90) (end 165.4767 90) (width 0.2) (layer "B.Cu") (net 22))
 (segment (start 184.3154 90.9767) (end 193.6687 100.33) (width 0.2) (layer "B.Cu") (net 22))
 (segment (start 182.8583 54.6115) (end 196.8485 54.6115) (width 0.2) (layer "B.Cu") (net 3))
 (segment (start 166.087 67.0233) (end 170.4465 67.0233) (width 0.2) (layer "B.Cu") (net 3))
 (segment (start 170.4465 67.0233) (end 182.8583 54.6115) (width 0.2) (layer "B.Cu") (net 3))
 (segment (start 165.4767 68) (end 165.4767 67.6336) (width 0.2) (layer "B.Cu") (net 3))
 (segment (start 165.4767 67.6336) (end 166.087 67.0233) (width 0.2) (layer "B.Cu") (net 3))
 (segment (start 164.5 68) (end 165.4767 68) (width 0.2) (layer "B.Cu") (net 3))
 (segment (start 196.8485 54.6115) (end 198.12 53.34) (width 0.2) (layer "B.Cu") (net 3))
 (segment (start 164.5 84) (end 165.4767 84) (width 0.2) (layer "B.Cu") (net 15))
 (segment (start 166.087 83.0233) (end 167.1217 83.0233) (width 0.2) (layer "B.Cu") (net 15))
 (segment (start 196.85 82.55) (end 198.12 81.28) (width 0.2) (layer "B.Cu") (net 15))
 (segment (start 165.4767 83.6336) (end 166.087 83.0233) (width 0.2) (layer "B.Cu") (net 15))
 (segment (start 167.595 82.55) (end 196.85 82.55) (width 0.2) (layer "B.Cu") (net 15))
 (segment (start 165.4767 84) (end 165.4767 83.6336) (width 0.2) (layer "B.Cu") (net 15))
 (segment (start 167.1217 83.0233) (end 167.595 82.55) (width 0.2) (layer "B.Cu") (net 15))
 (segment (start 166.1253 87.0149) (end 168.4229 87.0149) (width 0.2) (layer "B.Cu") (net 19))
 (segment (start 164.5 86) (end 165.4767 86) (width 0.2) (layer "B.Cu") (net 19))
 (segment (start 193.5432 92.71) (end 196.85 92.71) (width 0.2) (layer "B.Cu") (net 19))
 (segment (start 168.4229 87.0149) (end 169.4382 88.0302) (width 0.2) (layer "B.Cu") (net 19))
 (segment (start 196.85 92.71) (end 198.12 93.98) (width 0.2) (layer "B.Cu") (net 19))
 (segment (start 169.4382 88.0302) (end 188.8634 88.0302) (width 0.2) (layer "B.Cu") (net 19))
 (segment (start 165.4767 86) (end 165.4767 86.3663) (width 0.2) (layer "B.Cu") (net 19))
 (segment (start 165.4767 86.3663) (end 166.1253 87.0149) (width 0.2) (layer "B.Cu") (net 19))
 (segment (start 188.8634 88.0302) (end 193.5432 92.71) (width 0.2) (layer "B.Cu") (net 19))
 (segment (start 164.5 70) (end 165.4767 70) (width 0.2) (layer "B.Cu") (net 4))
 (segment (start 165.4767 69.6336) (end 165.4767 70) (width 0.2) (layer "B.Cu") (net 4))
 (segment (start 170.808 69.0233) (end 166.087 69.0233) (width 0.2) (layer "B.Cu") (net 4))
 (segment (start 196.8485 57.1515) (end 182.6798 57.1515) (width 0.2) (layer "B.Cu") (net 4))
 (segment (start 182.6798 57.1515) (end 170.808 69.0233) (width 0.2) (layer "B.Cu") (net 4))
 (segment (start 198.12 55.88) (end 196.8485 57.1515) (width 0.2) (layer "B.Cu") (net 4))
 (segment (start 166.087 69.0233) (end 165.4767 69.6336) (width 0.2) (layer "B.Cu") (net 4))
 (segment (start 196.85 95.25) (end 198.12 96.52) (width 0.2) (layer "B.Cu") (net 20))
 (segment (start 166.087 88.9767) (end 185.8331 88.9767) (width 0.2) (layer "B.Cu") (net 20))
 (segment (start 185.8331 88.9767) (end 192.1064 95.25) (width 0.2) (layer "B.Cu") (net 20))
 (segment (start 192.1064 95.25) (end 196.85 95.25) (width 0.2) (layer "B.Cu") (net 20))
 (segment (start 165.4767 88.3664) (end 166.087 88.9767) (width 0.2) (layer "B.Cu") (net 20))
 (segment (start 164.5 88) (end 165.4767 88) (width 0.2) (layer "B.Cu") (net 20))
 (segment (start 165.4767 88) (end 165.4767 88.3664) (width 0.2) (layer "B.Cu") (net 20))
 (segment (start 166.087 92.9767) (end 183.8292 92.9767) (width 0.2) (layer "B.Cu") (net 23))
 (segment (start 164.5 92) (end 165.4767 92) (width 0.2) (layer "B.Cu") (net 23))
 (segment (start 193.7225 102.87) (end 196.85 102.87) (width 0.2) (layer "B.Cu") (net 23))
 (segment (start 183.8292 92.9767) (end 193.7225 102.87) (width 0.2) (layer "B.Cu") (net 23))
 (segment (start 165.4767 92.3664) (end 166.087 92.9767) (width 0.2) (layer "B.Cu") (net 23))
 (segment (start 196.85 102.87) (end 198.12 104.14) (width 0.2) (layer "B.Cu") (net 23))
 (segment (start 165.4767 92) (end 165.4767 92.3664) (width 0.2) (layer "B.Cu") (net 23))
 (segment (start 182.7099 94.9767) (end 193.1432 105.41) (width 0.2) (layer "B.Cu") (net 24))
 (segment (start 166.087 94.9767) (end 182.7099 94.9767) (width 0.2) (layer "B.Cu") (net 24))
 (segment (start 164.5 94) (end 165.4767 94) (width 0.2) (layer "B.Cu") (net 24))
 (segment (start 196.85 105.41) (end 198.12 106.68) (width 0.2) (layer "B.Cu") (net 24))
 (segment (start 165.4767 94.3664) (end 166.087 94.9767) (width 0.2) (layer "B.Cu") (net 24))
 (segment (start 165.4767 94) (end 165.4767 94.3664) (width 0.2) (layer "B.Cu") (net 24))
 (segment (start 193.1432 105.41) (end 196.85 105.41) (width 0.2) (layer "B.Cu") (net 24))
 (segment (start 164.5 76) (end 165.4767 76) (width 0.2) (layer "B.Cu") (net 7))
 (segment (start 165.4767 75.6336) (end 166.087 75.0233) (width 0.2) (layer "B.Cu") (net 7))
 (segment (start 168.0198 75.0233) (end 178.2716 64.7715) (width 0.2) (layer "B.Cu") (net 7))
 (segment (start 196.8485 64.7715) (end 198.12 63.5) (width 0.2) (layer "B.Cu") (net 7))
 (segment (start 166.087 75.0233) (end 168.0198 75.0233) (width 0.2) (layer "B.Cu") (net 7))
 (segment (start 178.2716 64.7715) (end 196.8485 64.7715) (width 0.2) (layer "B.Cu") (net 7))
 (segment (start 165.4767 76) (end 165.4767 75.6336) (width 0.2) (layer "B.Cu") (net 7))
 (segment (start 196.85 107.95) (end 198.12 109.22) (width 0.2) (layer "B.Cu") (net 25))
 (segment (start 166.087 96.9767) (end 167.452 96.9767) (width 0.2) (layer "B.Cu") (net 25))
 (segment (start 165.4767 96) (end 165.4767 96.3664) (width 0.2) (layer "B.Cu") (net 25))
 (segment (start 178.4253 107.95) (end 196.85 107.95) (width 0.2) (layer "B.Cu") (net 25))
 (segment (start 167.452 96.9767) (end 178.4253 107.95) (width 0.2) (layer "B.Cu") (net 25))
 (segment (start 164.5 96) (end 165.4767 96) (width 0.2) (layer "B.Cu") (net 25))
 (segment (start 165.4767 96.3664) (end 166.087 96.9767) (width 0.2) (layer "B.Cu") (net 25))
 (segment (start 196.9549 112.9251) (end 198.12 111.76) (width 0.2) (layer "F.Cu") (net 26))
 (segment (start 167.4767 94) (end 186.4018 112.9251) (width 0.2) (layer "F.Cu") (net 26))
 (segment (start 186.4018 112.9251) (end 196.9549 112.9251) (width 0.2) (layer "F.Cu") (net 26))
 (segment (start 166.5 94) (end 167.4767 94) (width 0.2) (layer "F.Cu") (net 26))
 (segment (start 196.8485 69.8515) (end 198.12 68.58) (width 0.2) (layer "B.Cu") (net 9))
 (segment (start 164.5 80) (end 165.4767 80) (width 0.2) (layer "B.Cu") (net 9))
 (segment (start 166.087 79.0233) (end 168.0198 79.0233) (width 0.2) (layer "B.Cu") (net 9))
 (segment (start 177.1916 69.8515) (end 196.8485 69.8515) (width 0.2) (layer "B.Cu") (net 9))
 (segment (start 165.4767 79.6336) (end 166.087 79.0233) (width 0.2) (layer "B.Cu") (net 9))
 (segment (start 165.4767 80) (end 165.4767 79.6336) (width 0.2) (layer "B.Cu") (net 9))
 (segment (start 168.0198 79.0233) (end 177.1916 69.8515) (width 0.2) (layer "B.Cu") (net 9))
 (segment (start 165.4767 73.6336) (end 166.087 73.0233) (width 0.2) (layer "B.Cu") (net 6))
 (segment (start 180.7834 62.2315) (end 196.8485 62.2315) (width 0.2) (layer "B.Cu") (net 6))
 (segment (start 165.4767 74) (end 165.4767 73.6336) (width 0.2) (layer "B.Cu") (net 6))
 (segment (start 178.4186 64.0284) (end 178.9865 64.0284) (width 0.2) (layer "B.Cu") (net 6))
 (segment (start 164.5 74) (end 165.4767 74) (width 0.2) (layer "B.Cu") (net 6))
 (segment (start 178.9865 64.0284) (end 180.7834 62.2315) (width 0.2) (layer "B.Cu") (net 6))
 (segment (start 196.8485 62.2315) (end 198.12 60.96) (width 0.2) (layer "B.Cu") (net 6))
 (segment (start 166.087 73.0233) (end 169.4237 73.0233) (width 0.2) (layer "B.Cu") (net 6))
 (segment (start 169.4237 73.0233) (end 178.4186 64.0284) (width 0.2) (layer "B.Cu") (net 6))
 (segment (start 181.8684 72.3915) (end 196.8485 72.3915) (width 0.2) (layer "B.Cu") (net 10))
 (segment (start 165.4767 81.6336) (end 166.087 81.0233) (width 0.2) (layer "B.Cu") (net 10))
 (segment (start 173.2366 81.0233) (end 181.8684 72.3915) (width 0.2) (layer "B.Cu") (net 10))
 (segment (start 164.5 82) (end 165.4767 82) (width 0.2) (layer "B.Cu") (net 10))
 (segment (start 196.8485 72.3915) (end 198.12 71.12) (width 0.2) (layer "B.Cu") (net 10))
 (segment (start 166.087 81.0233) (end 173.2366 81.0233) (width 0.2) (layer "B.Cu") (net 10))
 (segment (start 165.4767 82) (end 165.4767 81.6336) (width 0.2) (layer "B.Cu") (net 10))
 (segment (start 166.087 71.0233) (end 169.376 71.0233) (width 0.2) (layer "B.Cu") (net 5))
 (segment (start 196.85 59.69) (end 198.12 58.42) (width 0.2) (layer "B.Cu") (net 5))
 (segment (start 164.5 72) (end 165.4767 72) (width 0.2) (layer "B.Cu") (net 5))
 (segment (start 176.914 63.4853) (end 178.8909 63.4853) (width 0.2) (layer "B.Cu") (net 5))
 (segment (start 182.6862 59.69) (end 196.85 59.69) (width 0.2) (layer "B.Cu") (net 5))
 (segment (start 169.376 71.0233) (end 176.914 63.4853) (width 0.2) (layer "B.Cu") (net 5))
 (segment (start 165.4767 71.6336) (end 166.087 71.0233) (width 0.2) (layer "B.Cu") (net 5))
 (segment (start 178.8909 63.4853) (end 182.6862 59.69) (width 0.2) (layer "B.Cu") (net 5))
 (segment (start 165.4767 72) (end 165.4767 71.6336) (width 0.2) (layer "B.Cu") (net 5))
 (segment (start 186.1077 90) (end 193.8977 97.79) (width 0.2) (layer "B.Cu") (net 21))
 (segment (start 166.5 90) (end 186.1077 90) (width 0.2) (layer "B.Cu") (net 21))
 (segment (start 193.8977 97.79) (end 196.85 97.79) (width 0.2) (layer "B.Cu") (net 21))
 (segment (start 196.85 97.79) (end 198.12 99.06) (width 0.2) (layer "B.Cu") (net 21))
 (segment (start 198.12 88.9) (end 196.8485 87.6285) (width 0.2) (layer "B.Cu") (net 18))
 (segment (start 196.8485 87.6285) (end 169.6753 87.6285) (width 0.2) (layer "B.Cu") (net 18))
 (segment (start 166.5 86) (end 167.4767 86) (width 0.2) (layer "B.Cu") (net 18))
 (segment (start 169.6753 87.6285) (end 168.0468 86) (width 0.2) (layer "B.Cu") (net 18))
 (segment (start 168.0468 86) (end 167.4767 86) (width 0.2) (layer "B.Cu") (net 18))
 (segment (start 166.087 77.0233) (end 168.0198 77.0233) (width 0.2) (layer "B.Cu") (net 8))
 (segment (start 165.4767 77.6336) (end 166.087 77.0233) (width 0.2) (layer "B.Cu") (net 8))
 (segment (start 177.7316 67.3115) (end 196.8485 67.3115) (width 0.2) (layer "B.Cu") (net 8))
 (segment (start 196.8485 67.3115) (end 198.12 66.04) (width 0.2) (layer "B.Cu") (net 8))
 (segment (start 164.5 78) (end 165.4767 78) (width 0.2) (layer "B.Cu") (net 8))
 (segment (start 168.0198 77.0233) (end 177.7316 67.3115) (width 0.2) (layer "B.Cu") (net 8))
 (segment (start 165.4767 78) (end 165.4767 77.6336) (width 0.2) (layer "B.Cu") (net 8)))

